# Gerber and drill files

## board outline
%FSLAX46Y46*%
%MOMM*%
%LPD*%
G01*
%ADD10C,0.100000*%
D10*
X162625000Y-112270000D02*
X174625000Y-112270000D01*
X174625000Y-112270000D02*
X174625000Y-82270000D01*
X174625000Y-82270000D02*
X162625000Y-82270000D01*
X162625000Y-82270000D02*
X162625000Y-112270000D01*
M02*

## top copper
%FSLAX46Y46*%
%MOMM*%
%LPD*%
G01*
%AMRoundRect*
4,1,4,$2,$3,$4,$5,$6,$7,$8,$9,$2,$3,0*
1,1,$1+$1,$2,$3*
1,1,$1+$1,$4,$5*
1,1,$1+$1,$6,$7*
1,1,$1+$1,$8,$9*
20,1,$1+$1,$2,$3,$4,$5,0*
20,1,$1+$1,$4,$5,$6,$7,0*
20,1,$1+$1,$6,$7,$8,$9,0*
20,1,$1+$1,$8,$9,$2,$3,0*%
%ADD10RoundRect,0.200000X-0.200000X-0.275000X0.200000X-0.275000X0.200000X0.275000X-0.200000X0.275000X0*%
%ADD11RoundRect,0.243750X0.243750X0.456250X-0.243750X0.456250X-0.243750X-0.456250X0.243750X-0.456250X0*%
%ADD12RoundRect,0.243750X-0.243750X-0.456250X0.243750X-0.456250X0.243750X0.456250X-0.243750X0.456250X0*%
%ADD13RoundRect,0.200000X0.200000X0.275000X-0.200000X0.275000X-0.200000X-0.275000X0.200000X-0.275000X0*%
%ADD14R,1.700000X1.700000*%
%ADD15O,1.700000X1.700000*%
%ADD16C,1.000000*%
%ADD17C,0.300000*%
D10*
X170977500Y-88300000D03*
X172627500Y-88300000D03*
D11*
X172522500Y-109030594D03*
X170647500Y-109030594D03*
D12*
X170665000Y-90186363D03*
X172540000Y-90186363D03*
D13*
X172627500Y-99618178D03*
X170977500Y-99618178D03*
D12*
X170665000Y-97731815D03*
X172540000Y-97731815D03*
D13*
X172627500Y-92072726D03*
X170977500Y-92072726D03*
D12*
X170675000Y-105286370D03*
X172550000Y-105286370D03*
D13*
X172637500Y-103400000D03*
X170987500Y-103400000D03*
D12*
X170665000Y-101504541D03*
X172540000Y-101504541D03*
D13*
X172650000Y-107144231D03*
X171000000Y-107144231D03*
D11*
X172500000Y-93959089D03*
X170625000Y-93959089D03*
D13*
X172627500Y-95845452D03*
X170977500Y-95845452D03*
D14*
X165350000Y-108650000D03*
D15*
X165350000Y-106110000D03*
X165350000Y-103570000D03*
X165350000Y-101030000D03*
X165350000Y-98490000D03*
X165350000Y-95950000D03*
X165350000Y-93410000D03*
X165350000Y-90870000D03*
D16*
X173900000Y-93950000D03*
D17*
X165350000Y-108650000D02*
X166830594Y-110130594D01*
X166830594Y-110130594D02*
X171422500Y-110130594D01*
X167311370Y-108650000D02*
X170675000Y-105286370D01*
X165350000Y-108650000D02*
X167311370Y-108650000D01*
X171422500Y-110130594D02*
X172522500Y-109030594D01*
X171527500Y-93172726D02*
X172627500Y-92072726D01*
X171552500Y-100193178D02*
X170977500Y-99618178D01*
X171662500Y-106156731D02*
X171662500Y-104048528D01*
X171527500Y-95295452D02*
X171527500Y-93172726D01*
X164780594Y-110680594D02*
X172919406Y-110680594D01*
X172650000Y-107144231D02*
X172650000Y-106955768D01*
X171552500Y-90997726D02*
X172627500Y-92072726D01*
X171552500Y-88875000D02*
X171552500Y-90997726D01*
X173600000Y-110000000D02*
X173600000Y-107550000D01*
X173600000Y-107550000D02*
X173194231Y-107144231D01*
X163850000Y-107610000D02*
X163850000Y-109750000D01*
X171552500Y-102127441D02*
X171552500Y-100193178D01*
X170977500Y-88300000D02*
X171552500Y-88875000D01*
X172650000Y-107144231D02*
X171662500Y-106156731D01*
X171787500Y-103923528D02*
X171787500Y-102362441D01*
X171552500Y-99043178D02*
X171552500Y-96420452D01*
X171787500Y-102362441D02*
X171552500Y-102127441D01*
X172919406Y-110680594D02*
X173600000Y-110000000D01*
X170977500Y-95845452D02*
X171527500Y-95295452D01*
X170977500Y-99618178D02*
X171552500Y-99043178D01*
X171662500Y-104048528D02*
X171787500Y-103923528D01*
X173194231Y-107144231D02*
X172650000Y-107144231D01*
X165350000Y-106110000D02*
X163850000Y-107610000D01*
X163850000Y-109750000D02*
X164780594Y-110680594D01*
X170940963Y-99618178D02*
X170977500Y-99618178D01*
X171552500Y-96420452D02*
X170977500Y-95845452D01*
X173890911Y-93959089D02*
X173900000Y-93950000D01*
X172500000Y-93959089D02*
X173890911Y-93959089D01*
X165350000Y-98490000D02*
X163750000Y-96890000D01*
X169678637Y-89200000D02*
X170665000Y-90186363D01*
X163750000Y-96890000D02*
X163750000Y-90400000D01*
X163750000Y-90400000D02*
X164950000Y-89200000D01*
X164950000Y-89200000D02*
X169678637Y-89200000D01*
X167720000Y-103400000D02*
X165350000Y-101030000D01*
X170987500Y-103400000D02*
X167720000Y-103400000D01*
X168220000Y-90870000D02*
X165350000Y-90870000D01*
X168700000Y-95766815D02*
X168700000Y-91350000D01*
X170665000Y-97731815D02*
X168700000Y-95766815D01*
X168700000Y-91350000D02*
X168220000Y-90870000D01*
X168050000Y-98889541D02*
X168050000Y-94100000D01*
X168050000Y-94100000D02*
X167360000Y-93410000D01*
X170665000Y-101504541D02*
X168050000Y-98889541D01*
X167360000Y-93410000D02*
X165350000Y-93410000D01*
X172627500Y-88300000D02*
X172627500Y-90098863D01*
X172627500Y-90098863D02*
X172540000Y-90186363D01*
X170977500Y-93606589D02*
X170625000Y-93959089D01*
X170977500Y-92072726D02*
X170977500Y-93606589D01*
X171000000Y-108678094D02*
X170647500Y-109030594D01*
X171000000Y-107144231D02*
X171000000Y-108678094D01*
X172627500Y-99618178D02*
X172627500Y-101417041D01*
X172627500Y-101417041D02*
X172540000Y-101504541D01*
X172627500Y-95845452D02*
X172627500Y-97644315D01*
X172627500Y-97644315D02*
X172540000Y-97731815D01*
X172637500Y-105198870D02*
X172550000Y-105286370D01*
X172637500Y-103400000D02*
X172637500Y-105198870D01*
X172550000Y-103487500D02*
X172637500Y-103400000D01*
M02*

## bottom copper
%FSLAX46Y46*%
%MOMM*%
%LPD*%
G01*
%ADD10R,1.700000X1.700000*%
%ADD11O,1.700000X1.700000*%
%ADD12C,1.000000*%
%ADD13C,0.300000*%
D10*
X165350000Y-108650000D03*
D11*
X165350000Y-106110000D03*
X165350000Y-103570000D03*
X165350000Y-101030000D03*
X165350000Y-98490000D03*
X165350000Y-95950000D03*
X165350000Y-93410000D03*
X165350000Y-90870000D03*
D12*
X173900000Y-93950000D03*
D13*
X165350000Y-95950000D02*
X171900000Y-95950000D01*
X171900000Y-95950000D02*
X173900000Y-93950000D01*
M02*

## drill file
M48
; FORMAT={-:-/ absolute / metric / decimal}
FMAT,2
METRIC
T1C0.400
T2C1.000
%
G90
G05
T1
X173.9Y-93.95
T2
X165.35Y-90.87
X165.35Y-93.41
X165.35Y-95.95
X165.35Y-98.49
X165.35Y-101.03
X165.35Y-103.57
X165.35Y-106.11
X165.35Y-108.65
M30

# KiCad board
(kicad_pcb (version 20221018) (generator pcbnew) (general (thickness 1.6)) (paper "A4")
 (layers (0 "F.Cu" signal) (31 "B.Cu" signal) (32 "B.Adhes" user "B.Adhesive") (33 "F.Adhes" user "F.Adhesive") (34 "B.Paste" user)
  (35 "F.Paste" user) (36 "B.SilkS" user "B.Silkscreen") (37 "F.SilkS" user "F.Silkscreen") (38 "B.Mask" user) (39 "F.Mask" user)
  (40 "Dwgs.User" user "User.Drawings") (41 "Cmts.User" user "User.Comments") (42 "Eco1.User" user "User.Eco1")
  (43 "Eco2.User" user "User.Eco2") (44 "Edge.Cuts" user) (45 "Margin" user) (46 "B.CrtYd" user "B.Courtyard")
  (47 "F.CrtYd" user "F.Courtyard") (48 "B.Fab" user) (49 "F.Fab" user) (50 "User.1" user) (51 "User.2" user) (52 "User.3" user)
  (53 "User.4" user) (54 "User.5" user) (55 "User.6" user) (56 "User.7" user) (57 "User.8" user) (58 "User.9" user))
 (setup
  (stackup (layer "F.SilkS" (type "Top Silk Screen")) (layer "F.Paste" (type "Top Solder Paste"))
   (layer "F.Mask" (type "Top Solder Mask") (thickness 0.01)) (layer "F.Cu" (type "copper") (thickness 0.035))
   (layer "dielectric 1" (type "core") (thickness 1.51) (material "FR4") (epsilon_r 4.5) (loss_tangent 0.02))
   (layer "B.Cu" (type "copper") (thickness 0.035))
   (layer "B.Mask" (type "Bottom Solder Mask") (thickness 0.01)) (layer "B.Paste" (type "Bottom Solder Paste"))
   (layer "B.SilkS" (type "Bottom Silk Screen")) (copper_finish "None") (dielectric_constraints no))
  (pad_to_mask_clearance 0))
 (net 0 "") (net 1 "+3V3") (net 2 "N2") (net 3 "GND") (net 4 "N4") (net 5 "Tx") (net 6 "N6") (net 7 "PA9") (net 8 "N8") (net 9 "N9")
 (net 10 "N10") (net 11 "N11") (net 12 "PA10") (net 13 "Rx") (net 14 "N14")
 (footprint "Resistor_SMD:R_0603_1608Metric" (layer "F.Cu") (at 171.8025 88.3)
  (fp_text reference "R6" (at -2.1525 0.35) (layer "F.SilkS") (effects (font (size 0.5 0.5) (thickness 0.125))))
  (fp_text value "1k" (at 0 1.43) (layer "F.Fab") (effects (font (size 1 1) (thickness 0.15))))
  (pad "1" smd roundrect (at -0.825 0) (size 0.8 0.95) (layers "F.Cu" "F.Paste" "F.Mask") (roundrect_rratio 0.25) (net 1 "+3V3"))
  (pad "2" smd roundrect (at 0.825 0) (size 0.8 0.95) (layers "F.Cu" "F.Paste" "F.Mask") (roundrect_rratio 0.25) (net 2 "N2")))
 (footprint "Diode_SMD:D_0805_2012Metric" (layer "F.Cu") (at 171.585 109.030594 180)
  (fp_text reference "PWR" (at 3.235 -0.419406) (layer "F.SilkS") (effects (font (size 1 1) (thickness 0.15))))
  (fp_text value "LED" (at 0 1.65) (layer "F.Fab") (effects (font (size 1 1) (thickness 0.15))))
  (pad "1" smd roundrect (at -0.9375 0 180) (size 0.975 1.4) (layers "F.Cu" "F.Paste" "F.Mask") (roundrect_rratio 0.25) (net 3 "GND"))
  (pad "2" smd roundrect (at 0.9375 0 180) (size 0.975 1.4) (layers "F.Cu" "F.Paste" "F.Mask") (roundrect_rratio 0.25) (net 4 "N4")))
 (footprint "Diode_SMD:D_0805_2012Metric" (layer "F.Cu") (at 171.6025 90.186363)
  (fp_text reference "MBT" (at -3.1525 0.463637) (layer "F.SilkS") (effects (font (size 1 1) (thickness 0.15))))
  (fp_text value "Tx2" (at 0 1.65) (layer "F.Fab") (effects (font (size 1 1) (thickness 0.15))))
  (pad "1" smd roundrect (at -0.9375 0) (size 0.975 1.4) (layers "F.Cu" "F.Paste" "F.Mask") (roundrect_rratio 0.25) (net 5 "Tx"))
  (pad "2" smd roundrect (at 0.9375 0) (size 0.975 1.4) (layers "F.Cu" "F.Paste" "F.Mask") (roundrect_rratio 0.25) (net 2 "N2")))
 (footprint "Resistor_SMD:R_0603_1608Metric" (layer "F.Cu") (at 171.8025 99.618178 180)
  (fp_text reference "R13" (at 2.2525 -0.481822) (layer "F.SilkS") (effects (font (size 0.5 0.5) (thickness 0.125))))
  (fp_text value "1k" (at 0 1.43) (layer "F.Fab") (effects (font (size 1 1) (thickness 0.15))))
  (pad "1" smd roundrect (at -0.825 0 180) (size 0.8 0.95) (layers "F.Cu" "F.Paste" "F.Mask") (roundrect_rratio 0.25) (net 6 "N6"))
  (pad "2" smd roundrect (at 0.825 0 180) (size 0.8 0.95) (layers "F.Cu" "F.Paste" "F.Mask") (roundrect_rratio 0.25) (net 1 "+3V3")))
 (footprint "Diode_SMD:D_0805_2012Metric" (layer "F.Cu") (at 171.6025 97.731815)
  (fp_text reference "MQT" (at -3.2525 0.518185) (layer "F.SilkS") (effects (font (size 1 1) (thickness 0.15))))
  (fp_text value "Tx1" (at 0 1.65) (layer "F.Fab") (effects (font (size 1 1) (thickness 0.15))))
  (pad "1" smd roundrect (at -0.9375 0) (size 0.975 1.4) (layers "F.Cu" "F.Paste" "F.Mask") (roundrect_rratio 0.25) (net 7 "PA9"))
  (pad "2" smd roundrect (at 0.9375 0) (size 0.975 1.4) (layers "F.Cu" "F.Paste" "F.Mask") (roundrect_rratio 0.25) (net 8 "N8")))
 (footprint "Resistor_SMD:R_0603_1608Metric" (layer "F.Cu") (at 171.8025 92.072726 180)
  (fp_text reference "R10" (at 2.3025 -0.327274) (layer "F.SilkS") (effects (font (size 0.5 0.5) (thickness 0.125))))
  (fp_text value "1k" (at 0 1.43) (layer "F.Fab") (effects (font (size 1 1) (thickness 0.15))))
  (pad "1" smd roundrect (at -0.825 0 180) (size 0.8 0.95) (layers "F.Cu" "F.Paste" "F.Mask") (roundrect_rratio 0.25) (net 1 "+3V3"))
  (pad "2" smd roundrect (at 0.825 0 180) (size 0.8 0.95) (layers "F.Cu" "F.Paste" "F.Mask") (roundrect_rratio 0.25) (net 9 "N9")))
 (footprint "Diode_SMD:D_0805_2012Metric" (layer "F.Cu") (at 171.6125 105.28637)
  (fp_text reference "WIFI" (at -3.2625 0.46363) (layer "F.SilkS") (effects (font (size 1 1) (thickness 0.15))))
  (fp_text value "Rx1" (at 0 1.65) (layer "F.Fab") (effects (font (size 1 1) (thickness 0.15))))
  (pad "1" smd roundrect (at -0.9375 0) (size 0.975 1.4) (layers "F.Cu" "F.Paste" "F.Mask") (roundrect_rratio 0.25) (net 3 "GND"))
  (pad "2" smd roundrect (at 0.9375 0) (size 0.975 1.4) (layers "F.Cu" "F.Paste" "F.Mask") (roundrect_rratio 0.25) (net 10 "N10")))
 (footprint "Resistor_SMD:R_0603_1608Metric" (layer "F.Cu") (at 171.8125 103.4 180)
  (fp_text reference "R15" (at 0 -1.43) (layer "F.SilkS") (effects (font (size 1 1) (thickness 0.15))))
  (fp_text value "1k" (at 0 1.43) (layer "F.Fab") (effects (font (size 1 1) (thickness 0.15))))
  (pad "1" smd roundrect (at -0.825 0 180) (size 0.8 0.95) (layers "F.Cu" "F.Paste" "F.Mask") (roundrect_rratio 0.25) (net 10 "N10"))
  (pad "2" smd roundrect (at 0.825 0 180) (size 0.8 0.95) (layers "F.Cu" "F.Paste" "F.Mask") (roundrect_rratio 0.25) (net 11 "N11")))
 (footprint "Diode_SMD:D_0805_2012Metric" (layer "F.Cu") (at 171.6025 101.504541)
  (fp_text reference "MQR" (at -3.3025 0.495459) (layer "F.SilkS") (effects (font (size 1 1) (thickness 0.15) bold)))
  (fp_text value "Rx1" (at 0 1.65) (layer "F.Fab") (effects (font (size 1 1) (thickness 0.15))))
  (pad "1" smd roundrect (at -0.9375 0) (size 0.975 1.4) (layers "F.Cu" "F.Paste" "F.Mask") (roundrect_rratio 0.25) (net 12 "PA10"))
  (pad "2" smd roundrect (at 0.9375 0) (size 0.975 1.4) (layers "F.Cu" "F.Paste" "F.Mask") (roundrect_rratio 0.25) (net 6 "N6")))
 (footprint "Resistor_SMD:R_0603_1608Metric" (layer "F.Cu") (at 171.825 107.144231 180)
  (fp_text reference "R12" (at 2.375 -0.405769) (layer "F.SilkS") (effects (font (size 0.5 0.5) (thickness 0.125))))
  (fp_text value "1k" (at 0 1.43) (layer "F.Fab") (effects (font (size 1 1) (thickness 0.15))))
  (pad "1" smd roundrect (at -0.825 0 180) (size 0.8 0.95) (layers "F.Cu" "F.Paste" "F.Mask") (roundrect_rratio 0.25) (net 1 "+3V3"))
  (pad "2" smd roundrect (at 0.825 0 180) (size 0.8 0.95) (layers "F.Cu" "F.Paste" "F.Mask") (roundrect_rratio 0.25) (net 4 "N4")))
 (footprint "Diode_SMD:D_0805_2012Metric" (layer "F.Cu") (at 171.5625 93.959089 180)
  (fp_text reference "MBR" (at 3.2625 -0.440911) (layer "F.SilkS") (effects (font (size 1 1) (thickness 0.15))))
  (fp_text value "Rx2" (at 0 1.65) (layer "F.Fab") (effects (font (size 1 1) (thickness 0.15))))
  (pad "1" smd roundrect (at -0.9375 0 180) (size 0.975 1.4) (layers "F.Cu" "F.Paste" "F.Mask") (roundrect_rratio 0.25) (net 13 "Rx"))
  (pad "2" smd roundrect (at 0.9375 0 180) (size 0.975 1.4) (layers "F.Cu" "F.Paste" "F.Mask") (roundrect_rratio 0.25) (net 9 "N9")))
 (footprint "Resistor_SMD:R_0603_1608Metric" (layer "F.Cu") (at 171.8025 95.845452 180)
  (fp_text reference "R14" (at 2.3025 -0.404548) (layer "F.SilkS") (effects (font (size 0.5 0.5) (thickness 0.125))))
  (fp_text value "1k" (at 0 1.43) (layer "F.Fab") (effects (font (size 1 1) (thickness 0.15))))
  (pad "1" smd roundrect (at -0.825 0 180) (size 0.8 0.95) (layers "F.Cu" "F.Paste" "F.Mask") (roundrect_rratio 0.25) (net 8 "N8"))
  (pad "2" smd roundrect (at 0.825 0 180) (size 0.8 0.95) (layers "F.Cu" "F.Paste" "F.Mask") (roundrect_rratio 0.25) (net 1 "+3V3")))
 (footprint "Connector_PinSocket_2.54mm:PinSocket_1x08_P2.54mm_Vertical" (layer "B.Cu") (at 165.35 108.65)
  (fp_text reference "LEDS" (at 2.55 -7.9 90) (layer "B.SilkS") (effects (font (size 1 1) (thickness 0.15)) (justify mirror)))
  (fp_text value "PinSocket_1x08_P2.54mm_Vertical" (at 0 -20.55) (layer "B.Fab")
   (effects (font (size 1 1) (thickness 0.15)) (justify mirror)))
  (pad "1" thru_hole rect (at 0 0) (size 1.7 1.7) (drill 1) (layers "*.Cu" "*.Mask") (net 3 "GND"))
  (pad "2" thru_hole oval (at 0 -2.54) (size 1.7 1.7) (drill 1) (layers "*.Cu" "*.Mask") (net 1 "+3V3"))
  (pad "3" thru_hole oval (at 0 -5.08) (size 1.7 1.7) (drill 1) (layers "*.Cu" "*.Mask") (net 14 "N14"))
  (pad "4" thru_hole oval (at 0 -7.62) (size 1.7 1.7) (drill 1) (layers "*.Cu" "*.Mask") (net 11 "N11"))
  (pad "5" thru_hole oval (at 0 -10.16) (size 1.7 1.7) (drill 1) (layers "*.Cu" "*.Mask") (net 5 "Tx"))
  (pad "6" thru_hole oval (at 0 -12.7) (size 1.7 1.7) (drill 1) (layers "*.Cu" "*.Mask") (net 13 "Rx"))
  (pad "7" thru_hole oval (at 0 -15.24) (size 1.7 1.7) (drill 1) (layers "*.Cu" "*.Mask") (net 12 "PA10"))
  (pad "8" thru_hole oval (at 0 -17.78) (size 1.7 1.7) (drill 1) (layers "*.Cu" "*.Mask") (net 7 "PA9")))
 (gr_line (start 162.625 112.27) (end 174.625 112.27) (stroke (width 0.1) (type solid)) (layer "Edge.Cuts"))
 (gr_line (start 174.625 112.27) (end 174.625 82.27) (stroke (width 0.1) (type solid)) (layer "Edge.Cuts"))
 (gr_line (start 174.625 82.27) (end 162.625 82.27) (stroke (width 0.1) (type solid)) (layer "Edge.Cuts"))
 (gr_line (start 162.625 82.27) (end 162.625 112.27) (stroke (width 0.1) (type solid)) (layer "Edge.Cuts"))
 (segment (start 165.35 108.65) (end 166.830594 110.130594) (width 0.3) (layer "F.Cu") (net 3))
 (segment (start 166.830594 110.130594) (end 171.4225 110.130594) (width 0.3) (layer "F.Cu") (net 3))
 (segment (start 167.31137 108.65) (end 170.675 105.28637) (width 0.3) (layer "F.Cu") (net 3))
 (segment (start 165.35 108.65) (end 167.31137 108.65) (width 0.3) (layer "F.Cu") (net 3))
 (segment (start 171.4225 110.130594) (end 172.5225 109.030594) (width 0.3) (layer "F.Cu") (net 3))
 (segment (start 171.5275 93.172726) (end 172.6275 92.072726) (width 0.3) (layer "F.Cu") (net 1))
 (segment (start 171.5525 100.193178) (end 170.9775 99.618178) (width 0.3) (layer "F.Cu") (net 1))
 (segment (start 171.6625 106.156731) (end 171.6625 104.048528) (width 0.3) (layer "F.Cu") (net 1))
 (segment (start 171.5275 95.295452) (end 171.5275 93.172726) (width 0.3) (layer "F.Cu") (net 1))
 (segment (start 164.780594 110.680594) (end 172.919406 110.680594) (width 0.3) (layer "F.Cu") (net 1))
 (segment (start 172.65 107.144231) (end 172.65 106.955768) (width 0.3) (layer "F.Cu") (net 1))
 (segment (start 171.5525 90.997726) (end 172.6275 92.072726) (width 0.3) (layer "F.Cu") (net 1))
 (segment (start 171.5525 88.875) (end 171.5525 90.997726) (width 0.3) (layer "F.Cu") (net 1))
 (segment (start 173.6 110) (end 173.6 107.55) (width 0.3) (layer "F.Cu") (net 1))
 (segment (start 173.6 107.55) (end 173.194231 107.144231) (width 0.3) (layer "F.Cu") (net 1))
 (segment (start 163.85 107.61) (end 163.85 109.75) (width 0.3) (layer "F.Cu") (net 1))
 (segment (start 171.5525 102.127441) (end 171.5525 100.193178) (width 0.3) (layer "F.Cu") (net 1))
 (segment (start 170.9775 88.3) (end 171.5525 88.875) (width 0.3) (layer "F.Cu") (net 1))
 (segment (start 172.65 107.144231) (end 171.6625 106.156731) (width 0.3) (layer "F.Cu") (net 1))
 (segment (start 171.7875 103.923528) (end 171.7875 102.362441) (width 0.3) (layer "F.Cu") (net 1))
 (segment (start 171.5525 99.043178) (end 171.5525 96.420452) (width 0.3) (layer "F.Cu") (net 1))
 (segment (start 171.7875 102.362441) (end 171.5525 102.127441) (width 0.3) (layer "F.Cu") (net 1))
 (segment (start 172.919406 110.680594) (end 173.6 110) (width 0.3) (layer "F.Cu") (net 1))
 (segment (start 170.9775 95.845452) (end 171.5275 95.295452) (width 0.3) (layer "F.Cu") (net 1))
 (segment (start 170.9775 99.618178) (end 171.5525 99.043178) (width 0.3) (layer "F.Cu") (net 1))
 (segment (start 171.6625 104.048528) (end 171.7875 103.923528) (width 0.3) (layer "F.Cu") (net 1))
 (segment (start 173.194231 107.144231) (end 172.65 107.144231) (width 0.3) (layer "F.Cu") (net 1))
 (segment (start 165.35 106.11) (end 163.85 107.61) (width 0.3) (layer "F.Cu") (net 1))
 (segment (start 163.85 109.75) (end 164.780594 110.680594) (width 0.3) (layer "F.Cu") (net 1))
 (segment (start 170.940963 99.618178) (end 170.9775 99.618178) (width 0.3) (layer "F.Cu") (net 1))
 (segment (start 171.5525 96.420452) (end 170.9775 95.845452) (width 0.3) (layer "F.Cu") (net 1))
 (segment (start 173.890911 93.959089) (end 173.9 93.95) (width 0.3) (layer "F.Cu") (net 13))
 (segment (start 172.5 93.959089) (end 173.890911 93.959089) (width 0.3) (layer "F.Cu") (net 13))
 (via (at 173.9 93.95) (size 1) (drill 0.4) (layers "F.Cu" "B.Cu") (free) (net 13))
 (segment (start 165.35 95.95) (end 171.9 95.95) (width 0.3) (layer "B.Cu") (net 13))
 (segment (start 171.9 95.95) (end 173.9 93.95) (width 0.3) (layer "B.Cu") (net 13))
 (segment (start 165.35 98.49) (end 163.75 96.89) (width 0.3) (layer "F.Cu") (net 5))
 (segment (start 169.678637 89.2) (end 170.665 90.186363) (width 0.3) (layer "F.Cu") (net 5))
 (segment (start 163.75 96.89) (end 163.75 90.4) (width 0.3) (layer "F.Cu") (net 5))
 (segment (start 163.75 90.4) (end 164.95 89.2) (width 0.3) (layer "F.Cu") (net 5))
 (segment (start 164.95 89.2) (end 169.678637 89.2) (width 0.3) (layer "F.Cu") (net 5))
 (segment (start 167.72 103.4) (end 165.35 101.03) (width 0.3) (layer "F.Cu") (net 11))
 (segment (start 170.9875 103.4) (end 167.72 103.4) (width 0.3) (layer "F.Cu") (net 11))
 (segment (start 168.22 90.87) (end 165.35 90.87) (width 0.3) (layer "F.Cu") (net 7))
 (segment (start 168.7 95.766815) (end 168.7 91.35) (width 0.3) (layer "F.Cu") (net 7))
 (segment (start 170.665 97.731815) (end 168.7 95.766815) (width 0.3) (layer "F.Cu") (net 7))
 (segment (start 168.7 91.35) (end 168.22 90.87) (width 0.3) (layer "F.Cu") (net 7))
 (segment (start 168.05 98.889541) (end 168.05 94.1) (width 0.3) (layer "F.Cu") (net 12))
 (segment (start 168.05 94.1) (end 167.36 93.41) (width 0.3) (layer "F.Cu") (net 12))
 (segment (start 170.665 101.504541) (end 168.05 98.889541) (width 0.3) (layer "F.Cu") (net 12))
 (segment (start 167.36 93.41) (end 165.35 93.41) (width 0.3) (layer "F.Cu") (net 12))
 (segment (start 172.6275 88.3) (end 172.6275 90.098863) (width 0.3) (layer "F.Cu") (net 2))
 (segment (start 172.6275 90.098863) (end 172.54 90.186363) (width 0.3) (layer "F.Cu") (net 2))
 (segment (start 170.9775 93.606589) (end 170.625 93.959089) (width 0.3) (layer "F.Cu") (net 9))
 (segment (start 170.9775 92.072726) (end 170.9775 93.606589) (width 0.3) (layer "F.Cu") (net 9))
 (segment (start 171 108.678094) (end 170.6475 109.030594) (width 0.3) (layer "F.Cu") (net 4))
 (segment (start 171 107.144231) (end 171 108.678094) (width 0.3) (layer "F.Cu") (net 4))
 (segment (start 172.6275 99.618178) (end 172.6275 101.417041) (width 0.3) (layer "F.Cu") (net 6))
 (segment (start 172.6275 101.417041) (end 172.54 101.504541) (width 0.3) (layer "F.Cu") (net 6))
 (segment (start 172.6275 95.845452) (end 172.6275 97.644315) (width 0.3) (layer "F.Cu") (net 8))
 (segment (start 172.6275 97.644315) (end 172.54 97.731815) (width 0.3) (layer "F.Cu") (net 8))
 (segment (start 172.6375 105.19887) (end 172.55 105.28637) (width 0.3) (layer "F.Cu") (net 10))
 (segment (start 172.6375 103.4) (end 172.6375 105.19887) (width 0.3) (layer "F.Cu") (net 10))
 (segment (start 172.55 103.4875) (end 172.6375 103.4) (width 0.3) (layer "F.Cu") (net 10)))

